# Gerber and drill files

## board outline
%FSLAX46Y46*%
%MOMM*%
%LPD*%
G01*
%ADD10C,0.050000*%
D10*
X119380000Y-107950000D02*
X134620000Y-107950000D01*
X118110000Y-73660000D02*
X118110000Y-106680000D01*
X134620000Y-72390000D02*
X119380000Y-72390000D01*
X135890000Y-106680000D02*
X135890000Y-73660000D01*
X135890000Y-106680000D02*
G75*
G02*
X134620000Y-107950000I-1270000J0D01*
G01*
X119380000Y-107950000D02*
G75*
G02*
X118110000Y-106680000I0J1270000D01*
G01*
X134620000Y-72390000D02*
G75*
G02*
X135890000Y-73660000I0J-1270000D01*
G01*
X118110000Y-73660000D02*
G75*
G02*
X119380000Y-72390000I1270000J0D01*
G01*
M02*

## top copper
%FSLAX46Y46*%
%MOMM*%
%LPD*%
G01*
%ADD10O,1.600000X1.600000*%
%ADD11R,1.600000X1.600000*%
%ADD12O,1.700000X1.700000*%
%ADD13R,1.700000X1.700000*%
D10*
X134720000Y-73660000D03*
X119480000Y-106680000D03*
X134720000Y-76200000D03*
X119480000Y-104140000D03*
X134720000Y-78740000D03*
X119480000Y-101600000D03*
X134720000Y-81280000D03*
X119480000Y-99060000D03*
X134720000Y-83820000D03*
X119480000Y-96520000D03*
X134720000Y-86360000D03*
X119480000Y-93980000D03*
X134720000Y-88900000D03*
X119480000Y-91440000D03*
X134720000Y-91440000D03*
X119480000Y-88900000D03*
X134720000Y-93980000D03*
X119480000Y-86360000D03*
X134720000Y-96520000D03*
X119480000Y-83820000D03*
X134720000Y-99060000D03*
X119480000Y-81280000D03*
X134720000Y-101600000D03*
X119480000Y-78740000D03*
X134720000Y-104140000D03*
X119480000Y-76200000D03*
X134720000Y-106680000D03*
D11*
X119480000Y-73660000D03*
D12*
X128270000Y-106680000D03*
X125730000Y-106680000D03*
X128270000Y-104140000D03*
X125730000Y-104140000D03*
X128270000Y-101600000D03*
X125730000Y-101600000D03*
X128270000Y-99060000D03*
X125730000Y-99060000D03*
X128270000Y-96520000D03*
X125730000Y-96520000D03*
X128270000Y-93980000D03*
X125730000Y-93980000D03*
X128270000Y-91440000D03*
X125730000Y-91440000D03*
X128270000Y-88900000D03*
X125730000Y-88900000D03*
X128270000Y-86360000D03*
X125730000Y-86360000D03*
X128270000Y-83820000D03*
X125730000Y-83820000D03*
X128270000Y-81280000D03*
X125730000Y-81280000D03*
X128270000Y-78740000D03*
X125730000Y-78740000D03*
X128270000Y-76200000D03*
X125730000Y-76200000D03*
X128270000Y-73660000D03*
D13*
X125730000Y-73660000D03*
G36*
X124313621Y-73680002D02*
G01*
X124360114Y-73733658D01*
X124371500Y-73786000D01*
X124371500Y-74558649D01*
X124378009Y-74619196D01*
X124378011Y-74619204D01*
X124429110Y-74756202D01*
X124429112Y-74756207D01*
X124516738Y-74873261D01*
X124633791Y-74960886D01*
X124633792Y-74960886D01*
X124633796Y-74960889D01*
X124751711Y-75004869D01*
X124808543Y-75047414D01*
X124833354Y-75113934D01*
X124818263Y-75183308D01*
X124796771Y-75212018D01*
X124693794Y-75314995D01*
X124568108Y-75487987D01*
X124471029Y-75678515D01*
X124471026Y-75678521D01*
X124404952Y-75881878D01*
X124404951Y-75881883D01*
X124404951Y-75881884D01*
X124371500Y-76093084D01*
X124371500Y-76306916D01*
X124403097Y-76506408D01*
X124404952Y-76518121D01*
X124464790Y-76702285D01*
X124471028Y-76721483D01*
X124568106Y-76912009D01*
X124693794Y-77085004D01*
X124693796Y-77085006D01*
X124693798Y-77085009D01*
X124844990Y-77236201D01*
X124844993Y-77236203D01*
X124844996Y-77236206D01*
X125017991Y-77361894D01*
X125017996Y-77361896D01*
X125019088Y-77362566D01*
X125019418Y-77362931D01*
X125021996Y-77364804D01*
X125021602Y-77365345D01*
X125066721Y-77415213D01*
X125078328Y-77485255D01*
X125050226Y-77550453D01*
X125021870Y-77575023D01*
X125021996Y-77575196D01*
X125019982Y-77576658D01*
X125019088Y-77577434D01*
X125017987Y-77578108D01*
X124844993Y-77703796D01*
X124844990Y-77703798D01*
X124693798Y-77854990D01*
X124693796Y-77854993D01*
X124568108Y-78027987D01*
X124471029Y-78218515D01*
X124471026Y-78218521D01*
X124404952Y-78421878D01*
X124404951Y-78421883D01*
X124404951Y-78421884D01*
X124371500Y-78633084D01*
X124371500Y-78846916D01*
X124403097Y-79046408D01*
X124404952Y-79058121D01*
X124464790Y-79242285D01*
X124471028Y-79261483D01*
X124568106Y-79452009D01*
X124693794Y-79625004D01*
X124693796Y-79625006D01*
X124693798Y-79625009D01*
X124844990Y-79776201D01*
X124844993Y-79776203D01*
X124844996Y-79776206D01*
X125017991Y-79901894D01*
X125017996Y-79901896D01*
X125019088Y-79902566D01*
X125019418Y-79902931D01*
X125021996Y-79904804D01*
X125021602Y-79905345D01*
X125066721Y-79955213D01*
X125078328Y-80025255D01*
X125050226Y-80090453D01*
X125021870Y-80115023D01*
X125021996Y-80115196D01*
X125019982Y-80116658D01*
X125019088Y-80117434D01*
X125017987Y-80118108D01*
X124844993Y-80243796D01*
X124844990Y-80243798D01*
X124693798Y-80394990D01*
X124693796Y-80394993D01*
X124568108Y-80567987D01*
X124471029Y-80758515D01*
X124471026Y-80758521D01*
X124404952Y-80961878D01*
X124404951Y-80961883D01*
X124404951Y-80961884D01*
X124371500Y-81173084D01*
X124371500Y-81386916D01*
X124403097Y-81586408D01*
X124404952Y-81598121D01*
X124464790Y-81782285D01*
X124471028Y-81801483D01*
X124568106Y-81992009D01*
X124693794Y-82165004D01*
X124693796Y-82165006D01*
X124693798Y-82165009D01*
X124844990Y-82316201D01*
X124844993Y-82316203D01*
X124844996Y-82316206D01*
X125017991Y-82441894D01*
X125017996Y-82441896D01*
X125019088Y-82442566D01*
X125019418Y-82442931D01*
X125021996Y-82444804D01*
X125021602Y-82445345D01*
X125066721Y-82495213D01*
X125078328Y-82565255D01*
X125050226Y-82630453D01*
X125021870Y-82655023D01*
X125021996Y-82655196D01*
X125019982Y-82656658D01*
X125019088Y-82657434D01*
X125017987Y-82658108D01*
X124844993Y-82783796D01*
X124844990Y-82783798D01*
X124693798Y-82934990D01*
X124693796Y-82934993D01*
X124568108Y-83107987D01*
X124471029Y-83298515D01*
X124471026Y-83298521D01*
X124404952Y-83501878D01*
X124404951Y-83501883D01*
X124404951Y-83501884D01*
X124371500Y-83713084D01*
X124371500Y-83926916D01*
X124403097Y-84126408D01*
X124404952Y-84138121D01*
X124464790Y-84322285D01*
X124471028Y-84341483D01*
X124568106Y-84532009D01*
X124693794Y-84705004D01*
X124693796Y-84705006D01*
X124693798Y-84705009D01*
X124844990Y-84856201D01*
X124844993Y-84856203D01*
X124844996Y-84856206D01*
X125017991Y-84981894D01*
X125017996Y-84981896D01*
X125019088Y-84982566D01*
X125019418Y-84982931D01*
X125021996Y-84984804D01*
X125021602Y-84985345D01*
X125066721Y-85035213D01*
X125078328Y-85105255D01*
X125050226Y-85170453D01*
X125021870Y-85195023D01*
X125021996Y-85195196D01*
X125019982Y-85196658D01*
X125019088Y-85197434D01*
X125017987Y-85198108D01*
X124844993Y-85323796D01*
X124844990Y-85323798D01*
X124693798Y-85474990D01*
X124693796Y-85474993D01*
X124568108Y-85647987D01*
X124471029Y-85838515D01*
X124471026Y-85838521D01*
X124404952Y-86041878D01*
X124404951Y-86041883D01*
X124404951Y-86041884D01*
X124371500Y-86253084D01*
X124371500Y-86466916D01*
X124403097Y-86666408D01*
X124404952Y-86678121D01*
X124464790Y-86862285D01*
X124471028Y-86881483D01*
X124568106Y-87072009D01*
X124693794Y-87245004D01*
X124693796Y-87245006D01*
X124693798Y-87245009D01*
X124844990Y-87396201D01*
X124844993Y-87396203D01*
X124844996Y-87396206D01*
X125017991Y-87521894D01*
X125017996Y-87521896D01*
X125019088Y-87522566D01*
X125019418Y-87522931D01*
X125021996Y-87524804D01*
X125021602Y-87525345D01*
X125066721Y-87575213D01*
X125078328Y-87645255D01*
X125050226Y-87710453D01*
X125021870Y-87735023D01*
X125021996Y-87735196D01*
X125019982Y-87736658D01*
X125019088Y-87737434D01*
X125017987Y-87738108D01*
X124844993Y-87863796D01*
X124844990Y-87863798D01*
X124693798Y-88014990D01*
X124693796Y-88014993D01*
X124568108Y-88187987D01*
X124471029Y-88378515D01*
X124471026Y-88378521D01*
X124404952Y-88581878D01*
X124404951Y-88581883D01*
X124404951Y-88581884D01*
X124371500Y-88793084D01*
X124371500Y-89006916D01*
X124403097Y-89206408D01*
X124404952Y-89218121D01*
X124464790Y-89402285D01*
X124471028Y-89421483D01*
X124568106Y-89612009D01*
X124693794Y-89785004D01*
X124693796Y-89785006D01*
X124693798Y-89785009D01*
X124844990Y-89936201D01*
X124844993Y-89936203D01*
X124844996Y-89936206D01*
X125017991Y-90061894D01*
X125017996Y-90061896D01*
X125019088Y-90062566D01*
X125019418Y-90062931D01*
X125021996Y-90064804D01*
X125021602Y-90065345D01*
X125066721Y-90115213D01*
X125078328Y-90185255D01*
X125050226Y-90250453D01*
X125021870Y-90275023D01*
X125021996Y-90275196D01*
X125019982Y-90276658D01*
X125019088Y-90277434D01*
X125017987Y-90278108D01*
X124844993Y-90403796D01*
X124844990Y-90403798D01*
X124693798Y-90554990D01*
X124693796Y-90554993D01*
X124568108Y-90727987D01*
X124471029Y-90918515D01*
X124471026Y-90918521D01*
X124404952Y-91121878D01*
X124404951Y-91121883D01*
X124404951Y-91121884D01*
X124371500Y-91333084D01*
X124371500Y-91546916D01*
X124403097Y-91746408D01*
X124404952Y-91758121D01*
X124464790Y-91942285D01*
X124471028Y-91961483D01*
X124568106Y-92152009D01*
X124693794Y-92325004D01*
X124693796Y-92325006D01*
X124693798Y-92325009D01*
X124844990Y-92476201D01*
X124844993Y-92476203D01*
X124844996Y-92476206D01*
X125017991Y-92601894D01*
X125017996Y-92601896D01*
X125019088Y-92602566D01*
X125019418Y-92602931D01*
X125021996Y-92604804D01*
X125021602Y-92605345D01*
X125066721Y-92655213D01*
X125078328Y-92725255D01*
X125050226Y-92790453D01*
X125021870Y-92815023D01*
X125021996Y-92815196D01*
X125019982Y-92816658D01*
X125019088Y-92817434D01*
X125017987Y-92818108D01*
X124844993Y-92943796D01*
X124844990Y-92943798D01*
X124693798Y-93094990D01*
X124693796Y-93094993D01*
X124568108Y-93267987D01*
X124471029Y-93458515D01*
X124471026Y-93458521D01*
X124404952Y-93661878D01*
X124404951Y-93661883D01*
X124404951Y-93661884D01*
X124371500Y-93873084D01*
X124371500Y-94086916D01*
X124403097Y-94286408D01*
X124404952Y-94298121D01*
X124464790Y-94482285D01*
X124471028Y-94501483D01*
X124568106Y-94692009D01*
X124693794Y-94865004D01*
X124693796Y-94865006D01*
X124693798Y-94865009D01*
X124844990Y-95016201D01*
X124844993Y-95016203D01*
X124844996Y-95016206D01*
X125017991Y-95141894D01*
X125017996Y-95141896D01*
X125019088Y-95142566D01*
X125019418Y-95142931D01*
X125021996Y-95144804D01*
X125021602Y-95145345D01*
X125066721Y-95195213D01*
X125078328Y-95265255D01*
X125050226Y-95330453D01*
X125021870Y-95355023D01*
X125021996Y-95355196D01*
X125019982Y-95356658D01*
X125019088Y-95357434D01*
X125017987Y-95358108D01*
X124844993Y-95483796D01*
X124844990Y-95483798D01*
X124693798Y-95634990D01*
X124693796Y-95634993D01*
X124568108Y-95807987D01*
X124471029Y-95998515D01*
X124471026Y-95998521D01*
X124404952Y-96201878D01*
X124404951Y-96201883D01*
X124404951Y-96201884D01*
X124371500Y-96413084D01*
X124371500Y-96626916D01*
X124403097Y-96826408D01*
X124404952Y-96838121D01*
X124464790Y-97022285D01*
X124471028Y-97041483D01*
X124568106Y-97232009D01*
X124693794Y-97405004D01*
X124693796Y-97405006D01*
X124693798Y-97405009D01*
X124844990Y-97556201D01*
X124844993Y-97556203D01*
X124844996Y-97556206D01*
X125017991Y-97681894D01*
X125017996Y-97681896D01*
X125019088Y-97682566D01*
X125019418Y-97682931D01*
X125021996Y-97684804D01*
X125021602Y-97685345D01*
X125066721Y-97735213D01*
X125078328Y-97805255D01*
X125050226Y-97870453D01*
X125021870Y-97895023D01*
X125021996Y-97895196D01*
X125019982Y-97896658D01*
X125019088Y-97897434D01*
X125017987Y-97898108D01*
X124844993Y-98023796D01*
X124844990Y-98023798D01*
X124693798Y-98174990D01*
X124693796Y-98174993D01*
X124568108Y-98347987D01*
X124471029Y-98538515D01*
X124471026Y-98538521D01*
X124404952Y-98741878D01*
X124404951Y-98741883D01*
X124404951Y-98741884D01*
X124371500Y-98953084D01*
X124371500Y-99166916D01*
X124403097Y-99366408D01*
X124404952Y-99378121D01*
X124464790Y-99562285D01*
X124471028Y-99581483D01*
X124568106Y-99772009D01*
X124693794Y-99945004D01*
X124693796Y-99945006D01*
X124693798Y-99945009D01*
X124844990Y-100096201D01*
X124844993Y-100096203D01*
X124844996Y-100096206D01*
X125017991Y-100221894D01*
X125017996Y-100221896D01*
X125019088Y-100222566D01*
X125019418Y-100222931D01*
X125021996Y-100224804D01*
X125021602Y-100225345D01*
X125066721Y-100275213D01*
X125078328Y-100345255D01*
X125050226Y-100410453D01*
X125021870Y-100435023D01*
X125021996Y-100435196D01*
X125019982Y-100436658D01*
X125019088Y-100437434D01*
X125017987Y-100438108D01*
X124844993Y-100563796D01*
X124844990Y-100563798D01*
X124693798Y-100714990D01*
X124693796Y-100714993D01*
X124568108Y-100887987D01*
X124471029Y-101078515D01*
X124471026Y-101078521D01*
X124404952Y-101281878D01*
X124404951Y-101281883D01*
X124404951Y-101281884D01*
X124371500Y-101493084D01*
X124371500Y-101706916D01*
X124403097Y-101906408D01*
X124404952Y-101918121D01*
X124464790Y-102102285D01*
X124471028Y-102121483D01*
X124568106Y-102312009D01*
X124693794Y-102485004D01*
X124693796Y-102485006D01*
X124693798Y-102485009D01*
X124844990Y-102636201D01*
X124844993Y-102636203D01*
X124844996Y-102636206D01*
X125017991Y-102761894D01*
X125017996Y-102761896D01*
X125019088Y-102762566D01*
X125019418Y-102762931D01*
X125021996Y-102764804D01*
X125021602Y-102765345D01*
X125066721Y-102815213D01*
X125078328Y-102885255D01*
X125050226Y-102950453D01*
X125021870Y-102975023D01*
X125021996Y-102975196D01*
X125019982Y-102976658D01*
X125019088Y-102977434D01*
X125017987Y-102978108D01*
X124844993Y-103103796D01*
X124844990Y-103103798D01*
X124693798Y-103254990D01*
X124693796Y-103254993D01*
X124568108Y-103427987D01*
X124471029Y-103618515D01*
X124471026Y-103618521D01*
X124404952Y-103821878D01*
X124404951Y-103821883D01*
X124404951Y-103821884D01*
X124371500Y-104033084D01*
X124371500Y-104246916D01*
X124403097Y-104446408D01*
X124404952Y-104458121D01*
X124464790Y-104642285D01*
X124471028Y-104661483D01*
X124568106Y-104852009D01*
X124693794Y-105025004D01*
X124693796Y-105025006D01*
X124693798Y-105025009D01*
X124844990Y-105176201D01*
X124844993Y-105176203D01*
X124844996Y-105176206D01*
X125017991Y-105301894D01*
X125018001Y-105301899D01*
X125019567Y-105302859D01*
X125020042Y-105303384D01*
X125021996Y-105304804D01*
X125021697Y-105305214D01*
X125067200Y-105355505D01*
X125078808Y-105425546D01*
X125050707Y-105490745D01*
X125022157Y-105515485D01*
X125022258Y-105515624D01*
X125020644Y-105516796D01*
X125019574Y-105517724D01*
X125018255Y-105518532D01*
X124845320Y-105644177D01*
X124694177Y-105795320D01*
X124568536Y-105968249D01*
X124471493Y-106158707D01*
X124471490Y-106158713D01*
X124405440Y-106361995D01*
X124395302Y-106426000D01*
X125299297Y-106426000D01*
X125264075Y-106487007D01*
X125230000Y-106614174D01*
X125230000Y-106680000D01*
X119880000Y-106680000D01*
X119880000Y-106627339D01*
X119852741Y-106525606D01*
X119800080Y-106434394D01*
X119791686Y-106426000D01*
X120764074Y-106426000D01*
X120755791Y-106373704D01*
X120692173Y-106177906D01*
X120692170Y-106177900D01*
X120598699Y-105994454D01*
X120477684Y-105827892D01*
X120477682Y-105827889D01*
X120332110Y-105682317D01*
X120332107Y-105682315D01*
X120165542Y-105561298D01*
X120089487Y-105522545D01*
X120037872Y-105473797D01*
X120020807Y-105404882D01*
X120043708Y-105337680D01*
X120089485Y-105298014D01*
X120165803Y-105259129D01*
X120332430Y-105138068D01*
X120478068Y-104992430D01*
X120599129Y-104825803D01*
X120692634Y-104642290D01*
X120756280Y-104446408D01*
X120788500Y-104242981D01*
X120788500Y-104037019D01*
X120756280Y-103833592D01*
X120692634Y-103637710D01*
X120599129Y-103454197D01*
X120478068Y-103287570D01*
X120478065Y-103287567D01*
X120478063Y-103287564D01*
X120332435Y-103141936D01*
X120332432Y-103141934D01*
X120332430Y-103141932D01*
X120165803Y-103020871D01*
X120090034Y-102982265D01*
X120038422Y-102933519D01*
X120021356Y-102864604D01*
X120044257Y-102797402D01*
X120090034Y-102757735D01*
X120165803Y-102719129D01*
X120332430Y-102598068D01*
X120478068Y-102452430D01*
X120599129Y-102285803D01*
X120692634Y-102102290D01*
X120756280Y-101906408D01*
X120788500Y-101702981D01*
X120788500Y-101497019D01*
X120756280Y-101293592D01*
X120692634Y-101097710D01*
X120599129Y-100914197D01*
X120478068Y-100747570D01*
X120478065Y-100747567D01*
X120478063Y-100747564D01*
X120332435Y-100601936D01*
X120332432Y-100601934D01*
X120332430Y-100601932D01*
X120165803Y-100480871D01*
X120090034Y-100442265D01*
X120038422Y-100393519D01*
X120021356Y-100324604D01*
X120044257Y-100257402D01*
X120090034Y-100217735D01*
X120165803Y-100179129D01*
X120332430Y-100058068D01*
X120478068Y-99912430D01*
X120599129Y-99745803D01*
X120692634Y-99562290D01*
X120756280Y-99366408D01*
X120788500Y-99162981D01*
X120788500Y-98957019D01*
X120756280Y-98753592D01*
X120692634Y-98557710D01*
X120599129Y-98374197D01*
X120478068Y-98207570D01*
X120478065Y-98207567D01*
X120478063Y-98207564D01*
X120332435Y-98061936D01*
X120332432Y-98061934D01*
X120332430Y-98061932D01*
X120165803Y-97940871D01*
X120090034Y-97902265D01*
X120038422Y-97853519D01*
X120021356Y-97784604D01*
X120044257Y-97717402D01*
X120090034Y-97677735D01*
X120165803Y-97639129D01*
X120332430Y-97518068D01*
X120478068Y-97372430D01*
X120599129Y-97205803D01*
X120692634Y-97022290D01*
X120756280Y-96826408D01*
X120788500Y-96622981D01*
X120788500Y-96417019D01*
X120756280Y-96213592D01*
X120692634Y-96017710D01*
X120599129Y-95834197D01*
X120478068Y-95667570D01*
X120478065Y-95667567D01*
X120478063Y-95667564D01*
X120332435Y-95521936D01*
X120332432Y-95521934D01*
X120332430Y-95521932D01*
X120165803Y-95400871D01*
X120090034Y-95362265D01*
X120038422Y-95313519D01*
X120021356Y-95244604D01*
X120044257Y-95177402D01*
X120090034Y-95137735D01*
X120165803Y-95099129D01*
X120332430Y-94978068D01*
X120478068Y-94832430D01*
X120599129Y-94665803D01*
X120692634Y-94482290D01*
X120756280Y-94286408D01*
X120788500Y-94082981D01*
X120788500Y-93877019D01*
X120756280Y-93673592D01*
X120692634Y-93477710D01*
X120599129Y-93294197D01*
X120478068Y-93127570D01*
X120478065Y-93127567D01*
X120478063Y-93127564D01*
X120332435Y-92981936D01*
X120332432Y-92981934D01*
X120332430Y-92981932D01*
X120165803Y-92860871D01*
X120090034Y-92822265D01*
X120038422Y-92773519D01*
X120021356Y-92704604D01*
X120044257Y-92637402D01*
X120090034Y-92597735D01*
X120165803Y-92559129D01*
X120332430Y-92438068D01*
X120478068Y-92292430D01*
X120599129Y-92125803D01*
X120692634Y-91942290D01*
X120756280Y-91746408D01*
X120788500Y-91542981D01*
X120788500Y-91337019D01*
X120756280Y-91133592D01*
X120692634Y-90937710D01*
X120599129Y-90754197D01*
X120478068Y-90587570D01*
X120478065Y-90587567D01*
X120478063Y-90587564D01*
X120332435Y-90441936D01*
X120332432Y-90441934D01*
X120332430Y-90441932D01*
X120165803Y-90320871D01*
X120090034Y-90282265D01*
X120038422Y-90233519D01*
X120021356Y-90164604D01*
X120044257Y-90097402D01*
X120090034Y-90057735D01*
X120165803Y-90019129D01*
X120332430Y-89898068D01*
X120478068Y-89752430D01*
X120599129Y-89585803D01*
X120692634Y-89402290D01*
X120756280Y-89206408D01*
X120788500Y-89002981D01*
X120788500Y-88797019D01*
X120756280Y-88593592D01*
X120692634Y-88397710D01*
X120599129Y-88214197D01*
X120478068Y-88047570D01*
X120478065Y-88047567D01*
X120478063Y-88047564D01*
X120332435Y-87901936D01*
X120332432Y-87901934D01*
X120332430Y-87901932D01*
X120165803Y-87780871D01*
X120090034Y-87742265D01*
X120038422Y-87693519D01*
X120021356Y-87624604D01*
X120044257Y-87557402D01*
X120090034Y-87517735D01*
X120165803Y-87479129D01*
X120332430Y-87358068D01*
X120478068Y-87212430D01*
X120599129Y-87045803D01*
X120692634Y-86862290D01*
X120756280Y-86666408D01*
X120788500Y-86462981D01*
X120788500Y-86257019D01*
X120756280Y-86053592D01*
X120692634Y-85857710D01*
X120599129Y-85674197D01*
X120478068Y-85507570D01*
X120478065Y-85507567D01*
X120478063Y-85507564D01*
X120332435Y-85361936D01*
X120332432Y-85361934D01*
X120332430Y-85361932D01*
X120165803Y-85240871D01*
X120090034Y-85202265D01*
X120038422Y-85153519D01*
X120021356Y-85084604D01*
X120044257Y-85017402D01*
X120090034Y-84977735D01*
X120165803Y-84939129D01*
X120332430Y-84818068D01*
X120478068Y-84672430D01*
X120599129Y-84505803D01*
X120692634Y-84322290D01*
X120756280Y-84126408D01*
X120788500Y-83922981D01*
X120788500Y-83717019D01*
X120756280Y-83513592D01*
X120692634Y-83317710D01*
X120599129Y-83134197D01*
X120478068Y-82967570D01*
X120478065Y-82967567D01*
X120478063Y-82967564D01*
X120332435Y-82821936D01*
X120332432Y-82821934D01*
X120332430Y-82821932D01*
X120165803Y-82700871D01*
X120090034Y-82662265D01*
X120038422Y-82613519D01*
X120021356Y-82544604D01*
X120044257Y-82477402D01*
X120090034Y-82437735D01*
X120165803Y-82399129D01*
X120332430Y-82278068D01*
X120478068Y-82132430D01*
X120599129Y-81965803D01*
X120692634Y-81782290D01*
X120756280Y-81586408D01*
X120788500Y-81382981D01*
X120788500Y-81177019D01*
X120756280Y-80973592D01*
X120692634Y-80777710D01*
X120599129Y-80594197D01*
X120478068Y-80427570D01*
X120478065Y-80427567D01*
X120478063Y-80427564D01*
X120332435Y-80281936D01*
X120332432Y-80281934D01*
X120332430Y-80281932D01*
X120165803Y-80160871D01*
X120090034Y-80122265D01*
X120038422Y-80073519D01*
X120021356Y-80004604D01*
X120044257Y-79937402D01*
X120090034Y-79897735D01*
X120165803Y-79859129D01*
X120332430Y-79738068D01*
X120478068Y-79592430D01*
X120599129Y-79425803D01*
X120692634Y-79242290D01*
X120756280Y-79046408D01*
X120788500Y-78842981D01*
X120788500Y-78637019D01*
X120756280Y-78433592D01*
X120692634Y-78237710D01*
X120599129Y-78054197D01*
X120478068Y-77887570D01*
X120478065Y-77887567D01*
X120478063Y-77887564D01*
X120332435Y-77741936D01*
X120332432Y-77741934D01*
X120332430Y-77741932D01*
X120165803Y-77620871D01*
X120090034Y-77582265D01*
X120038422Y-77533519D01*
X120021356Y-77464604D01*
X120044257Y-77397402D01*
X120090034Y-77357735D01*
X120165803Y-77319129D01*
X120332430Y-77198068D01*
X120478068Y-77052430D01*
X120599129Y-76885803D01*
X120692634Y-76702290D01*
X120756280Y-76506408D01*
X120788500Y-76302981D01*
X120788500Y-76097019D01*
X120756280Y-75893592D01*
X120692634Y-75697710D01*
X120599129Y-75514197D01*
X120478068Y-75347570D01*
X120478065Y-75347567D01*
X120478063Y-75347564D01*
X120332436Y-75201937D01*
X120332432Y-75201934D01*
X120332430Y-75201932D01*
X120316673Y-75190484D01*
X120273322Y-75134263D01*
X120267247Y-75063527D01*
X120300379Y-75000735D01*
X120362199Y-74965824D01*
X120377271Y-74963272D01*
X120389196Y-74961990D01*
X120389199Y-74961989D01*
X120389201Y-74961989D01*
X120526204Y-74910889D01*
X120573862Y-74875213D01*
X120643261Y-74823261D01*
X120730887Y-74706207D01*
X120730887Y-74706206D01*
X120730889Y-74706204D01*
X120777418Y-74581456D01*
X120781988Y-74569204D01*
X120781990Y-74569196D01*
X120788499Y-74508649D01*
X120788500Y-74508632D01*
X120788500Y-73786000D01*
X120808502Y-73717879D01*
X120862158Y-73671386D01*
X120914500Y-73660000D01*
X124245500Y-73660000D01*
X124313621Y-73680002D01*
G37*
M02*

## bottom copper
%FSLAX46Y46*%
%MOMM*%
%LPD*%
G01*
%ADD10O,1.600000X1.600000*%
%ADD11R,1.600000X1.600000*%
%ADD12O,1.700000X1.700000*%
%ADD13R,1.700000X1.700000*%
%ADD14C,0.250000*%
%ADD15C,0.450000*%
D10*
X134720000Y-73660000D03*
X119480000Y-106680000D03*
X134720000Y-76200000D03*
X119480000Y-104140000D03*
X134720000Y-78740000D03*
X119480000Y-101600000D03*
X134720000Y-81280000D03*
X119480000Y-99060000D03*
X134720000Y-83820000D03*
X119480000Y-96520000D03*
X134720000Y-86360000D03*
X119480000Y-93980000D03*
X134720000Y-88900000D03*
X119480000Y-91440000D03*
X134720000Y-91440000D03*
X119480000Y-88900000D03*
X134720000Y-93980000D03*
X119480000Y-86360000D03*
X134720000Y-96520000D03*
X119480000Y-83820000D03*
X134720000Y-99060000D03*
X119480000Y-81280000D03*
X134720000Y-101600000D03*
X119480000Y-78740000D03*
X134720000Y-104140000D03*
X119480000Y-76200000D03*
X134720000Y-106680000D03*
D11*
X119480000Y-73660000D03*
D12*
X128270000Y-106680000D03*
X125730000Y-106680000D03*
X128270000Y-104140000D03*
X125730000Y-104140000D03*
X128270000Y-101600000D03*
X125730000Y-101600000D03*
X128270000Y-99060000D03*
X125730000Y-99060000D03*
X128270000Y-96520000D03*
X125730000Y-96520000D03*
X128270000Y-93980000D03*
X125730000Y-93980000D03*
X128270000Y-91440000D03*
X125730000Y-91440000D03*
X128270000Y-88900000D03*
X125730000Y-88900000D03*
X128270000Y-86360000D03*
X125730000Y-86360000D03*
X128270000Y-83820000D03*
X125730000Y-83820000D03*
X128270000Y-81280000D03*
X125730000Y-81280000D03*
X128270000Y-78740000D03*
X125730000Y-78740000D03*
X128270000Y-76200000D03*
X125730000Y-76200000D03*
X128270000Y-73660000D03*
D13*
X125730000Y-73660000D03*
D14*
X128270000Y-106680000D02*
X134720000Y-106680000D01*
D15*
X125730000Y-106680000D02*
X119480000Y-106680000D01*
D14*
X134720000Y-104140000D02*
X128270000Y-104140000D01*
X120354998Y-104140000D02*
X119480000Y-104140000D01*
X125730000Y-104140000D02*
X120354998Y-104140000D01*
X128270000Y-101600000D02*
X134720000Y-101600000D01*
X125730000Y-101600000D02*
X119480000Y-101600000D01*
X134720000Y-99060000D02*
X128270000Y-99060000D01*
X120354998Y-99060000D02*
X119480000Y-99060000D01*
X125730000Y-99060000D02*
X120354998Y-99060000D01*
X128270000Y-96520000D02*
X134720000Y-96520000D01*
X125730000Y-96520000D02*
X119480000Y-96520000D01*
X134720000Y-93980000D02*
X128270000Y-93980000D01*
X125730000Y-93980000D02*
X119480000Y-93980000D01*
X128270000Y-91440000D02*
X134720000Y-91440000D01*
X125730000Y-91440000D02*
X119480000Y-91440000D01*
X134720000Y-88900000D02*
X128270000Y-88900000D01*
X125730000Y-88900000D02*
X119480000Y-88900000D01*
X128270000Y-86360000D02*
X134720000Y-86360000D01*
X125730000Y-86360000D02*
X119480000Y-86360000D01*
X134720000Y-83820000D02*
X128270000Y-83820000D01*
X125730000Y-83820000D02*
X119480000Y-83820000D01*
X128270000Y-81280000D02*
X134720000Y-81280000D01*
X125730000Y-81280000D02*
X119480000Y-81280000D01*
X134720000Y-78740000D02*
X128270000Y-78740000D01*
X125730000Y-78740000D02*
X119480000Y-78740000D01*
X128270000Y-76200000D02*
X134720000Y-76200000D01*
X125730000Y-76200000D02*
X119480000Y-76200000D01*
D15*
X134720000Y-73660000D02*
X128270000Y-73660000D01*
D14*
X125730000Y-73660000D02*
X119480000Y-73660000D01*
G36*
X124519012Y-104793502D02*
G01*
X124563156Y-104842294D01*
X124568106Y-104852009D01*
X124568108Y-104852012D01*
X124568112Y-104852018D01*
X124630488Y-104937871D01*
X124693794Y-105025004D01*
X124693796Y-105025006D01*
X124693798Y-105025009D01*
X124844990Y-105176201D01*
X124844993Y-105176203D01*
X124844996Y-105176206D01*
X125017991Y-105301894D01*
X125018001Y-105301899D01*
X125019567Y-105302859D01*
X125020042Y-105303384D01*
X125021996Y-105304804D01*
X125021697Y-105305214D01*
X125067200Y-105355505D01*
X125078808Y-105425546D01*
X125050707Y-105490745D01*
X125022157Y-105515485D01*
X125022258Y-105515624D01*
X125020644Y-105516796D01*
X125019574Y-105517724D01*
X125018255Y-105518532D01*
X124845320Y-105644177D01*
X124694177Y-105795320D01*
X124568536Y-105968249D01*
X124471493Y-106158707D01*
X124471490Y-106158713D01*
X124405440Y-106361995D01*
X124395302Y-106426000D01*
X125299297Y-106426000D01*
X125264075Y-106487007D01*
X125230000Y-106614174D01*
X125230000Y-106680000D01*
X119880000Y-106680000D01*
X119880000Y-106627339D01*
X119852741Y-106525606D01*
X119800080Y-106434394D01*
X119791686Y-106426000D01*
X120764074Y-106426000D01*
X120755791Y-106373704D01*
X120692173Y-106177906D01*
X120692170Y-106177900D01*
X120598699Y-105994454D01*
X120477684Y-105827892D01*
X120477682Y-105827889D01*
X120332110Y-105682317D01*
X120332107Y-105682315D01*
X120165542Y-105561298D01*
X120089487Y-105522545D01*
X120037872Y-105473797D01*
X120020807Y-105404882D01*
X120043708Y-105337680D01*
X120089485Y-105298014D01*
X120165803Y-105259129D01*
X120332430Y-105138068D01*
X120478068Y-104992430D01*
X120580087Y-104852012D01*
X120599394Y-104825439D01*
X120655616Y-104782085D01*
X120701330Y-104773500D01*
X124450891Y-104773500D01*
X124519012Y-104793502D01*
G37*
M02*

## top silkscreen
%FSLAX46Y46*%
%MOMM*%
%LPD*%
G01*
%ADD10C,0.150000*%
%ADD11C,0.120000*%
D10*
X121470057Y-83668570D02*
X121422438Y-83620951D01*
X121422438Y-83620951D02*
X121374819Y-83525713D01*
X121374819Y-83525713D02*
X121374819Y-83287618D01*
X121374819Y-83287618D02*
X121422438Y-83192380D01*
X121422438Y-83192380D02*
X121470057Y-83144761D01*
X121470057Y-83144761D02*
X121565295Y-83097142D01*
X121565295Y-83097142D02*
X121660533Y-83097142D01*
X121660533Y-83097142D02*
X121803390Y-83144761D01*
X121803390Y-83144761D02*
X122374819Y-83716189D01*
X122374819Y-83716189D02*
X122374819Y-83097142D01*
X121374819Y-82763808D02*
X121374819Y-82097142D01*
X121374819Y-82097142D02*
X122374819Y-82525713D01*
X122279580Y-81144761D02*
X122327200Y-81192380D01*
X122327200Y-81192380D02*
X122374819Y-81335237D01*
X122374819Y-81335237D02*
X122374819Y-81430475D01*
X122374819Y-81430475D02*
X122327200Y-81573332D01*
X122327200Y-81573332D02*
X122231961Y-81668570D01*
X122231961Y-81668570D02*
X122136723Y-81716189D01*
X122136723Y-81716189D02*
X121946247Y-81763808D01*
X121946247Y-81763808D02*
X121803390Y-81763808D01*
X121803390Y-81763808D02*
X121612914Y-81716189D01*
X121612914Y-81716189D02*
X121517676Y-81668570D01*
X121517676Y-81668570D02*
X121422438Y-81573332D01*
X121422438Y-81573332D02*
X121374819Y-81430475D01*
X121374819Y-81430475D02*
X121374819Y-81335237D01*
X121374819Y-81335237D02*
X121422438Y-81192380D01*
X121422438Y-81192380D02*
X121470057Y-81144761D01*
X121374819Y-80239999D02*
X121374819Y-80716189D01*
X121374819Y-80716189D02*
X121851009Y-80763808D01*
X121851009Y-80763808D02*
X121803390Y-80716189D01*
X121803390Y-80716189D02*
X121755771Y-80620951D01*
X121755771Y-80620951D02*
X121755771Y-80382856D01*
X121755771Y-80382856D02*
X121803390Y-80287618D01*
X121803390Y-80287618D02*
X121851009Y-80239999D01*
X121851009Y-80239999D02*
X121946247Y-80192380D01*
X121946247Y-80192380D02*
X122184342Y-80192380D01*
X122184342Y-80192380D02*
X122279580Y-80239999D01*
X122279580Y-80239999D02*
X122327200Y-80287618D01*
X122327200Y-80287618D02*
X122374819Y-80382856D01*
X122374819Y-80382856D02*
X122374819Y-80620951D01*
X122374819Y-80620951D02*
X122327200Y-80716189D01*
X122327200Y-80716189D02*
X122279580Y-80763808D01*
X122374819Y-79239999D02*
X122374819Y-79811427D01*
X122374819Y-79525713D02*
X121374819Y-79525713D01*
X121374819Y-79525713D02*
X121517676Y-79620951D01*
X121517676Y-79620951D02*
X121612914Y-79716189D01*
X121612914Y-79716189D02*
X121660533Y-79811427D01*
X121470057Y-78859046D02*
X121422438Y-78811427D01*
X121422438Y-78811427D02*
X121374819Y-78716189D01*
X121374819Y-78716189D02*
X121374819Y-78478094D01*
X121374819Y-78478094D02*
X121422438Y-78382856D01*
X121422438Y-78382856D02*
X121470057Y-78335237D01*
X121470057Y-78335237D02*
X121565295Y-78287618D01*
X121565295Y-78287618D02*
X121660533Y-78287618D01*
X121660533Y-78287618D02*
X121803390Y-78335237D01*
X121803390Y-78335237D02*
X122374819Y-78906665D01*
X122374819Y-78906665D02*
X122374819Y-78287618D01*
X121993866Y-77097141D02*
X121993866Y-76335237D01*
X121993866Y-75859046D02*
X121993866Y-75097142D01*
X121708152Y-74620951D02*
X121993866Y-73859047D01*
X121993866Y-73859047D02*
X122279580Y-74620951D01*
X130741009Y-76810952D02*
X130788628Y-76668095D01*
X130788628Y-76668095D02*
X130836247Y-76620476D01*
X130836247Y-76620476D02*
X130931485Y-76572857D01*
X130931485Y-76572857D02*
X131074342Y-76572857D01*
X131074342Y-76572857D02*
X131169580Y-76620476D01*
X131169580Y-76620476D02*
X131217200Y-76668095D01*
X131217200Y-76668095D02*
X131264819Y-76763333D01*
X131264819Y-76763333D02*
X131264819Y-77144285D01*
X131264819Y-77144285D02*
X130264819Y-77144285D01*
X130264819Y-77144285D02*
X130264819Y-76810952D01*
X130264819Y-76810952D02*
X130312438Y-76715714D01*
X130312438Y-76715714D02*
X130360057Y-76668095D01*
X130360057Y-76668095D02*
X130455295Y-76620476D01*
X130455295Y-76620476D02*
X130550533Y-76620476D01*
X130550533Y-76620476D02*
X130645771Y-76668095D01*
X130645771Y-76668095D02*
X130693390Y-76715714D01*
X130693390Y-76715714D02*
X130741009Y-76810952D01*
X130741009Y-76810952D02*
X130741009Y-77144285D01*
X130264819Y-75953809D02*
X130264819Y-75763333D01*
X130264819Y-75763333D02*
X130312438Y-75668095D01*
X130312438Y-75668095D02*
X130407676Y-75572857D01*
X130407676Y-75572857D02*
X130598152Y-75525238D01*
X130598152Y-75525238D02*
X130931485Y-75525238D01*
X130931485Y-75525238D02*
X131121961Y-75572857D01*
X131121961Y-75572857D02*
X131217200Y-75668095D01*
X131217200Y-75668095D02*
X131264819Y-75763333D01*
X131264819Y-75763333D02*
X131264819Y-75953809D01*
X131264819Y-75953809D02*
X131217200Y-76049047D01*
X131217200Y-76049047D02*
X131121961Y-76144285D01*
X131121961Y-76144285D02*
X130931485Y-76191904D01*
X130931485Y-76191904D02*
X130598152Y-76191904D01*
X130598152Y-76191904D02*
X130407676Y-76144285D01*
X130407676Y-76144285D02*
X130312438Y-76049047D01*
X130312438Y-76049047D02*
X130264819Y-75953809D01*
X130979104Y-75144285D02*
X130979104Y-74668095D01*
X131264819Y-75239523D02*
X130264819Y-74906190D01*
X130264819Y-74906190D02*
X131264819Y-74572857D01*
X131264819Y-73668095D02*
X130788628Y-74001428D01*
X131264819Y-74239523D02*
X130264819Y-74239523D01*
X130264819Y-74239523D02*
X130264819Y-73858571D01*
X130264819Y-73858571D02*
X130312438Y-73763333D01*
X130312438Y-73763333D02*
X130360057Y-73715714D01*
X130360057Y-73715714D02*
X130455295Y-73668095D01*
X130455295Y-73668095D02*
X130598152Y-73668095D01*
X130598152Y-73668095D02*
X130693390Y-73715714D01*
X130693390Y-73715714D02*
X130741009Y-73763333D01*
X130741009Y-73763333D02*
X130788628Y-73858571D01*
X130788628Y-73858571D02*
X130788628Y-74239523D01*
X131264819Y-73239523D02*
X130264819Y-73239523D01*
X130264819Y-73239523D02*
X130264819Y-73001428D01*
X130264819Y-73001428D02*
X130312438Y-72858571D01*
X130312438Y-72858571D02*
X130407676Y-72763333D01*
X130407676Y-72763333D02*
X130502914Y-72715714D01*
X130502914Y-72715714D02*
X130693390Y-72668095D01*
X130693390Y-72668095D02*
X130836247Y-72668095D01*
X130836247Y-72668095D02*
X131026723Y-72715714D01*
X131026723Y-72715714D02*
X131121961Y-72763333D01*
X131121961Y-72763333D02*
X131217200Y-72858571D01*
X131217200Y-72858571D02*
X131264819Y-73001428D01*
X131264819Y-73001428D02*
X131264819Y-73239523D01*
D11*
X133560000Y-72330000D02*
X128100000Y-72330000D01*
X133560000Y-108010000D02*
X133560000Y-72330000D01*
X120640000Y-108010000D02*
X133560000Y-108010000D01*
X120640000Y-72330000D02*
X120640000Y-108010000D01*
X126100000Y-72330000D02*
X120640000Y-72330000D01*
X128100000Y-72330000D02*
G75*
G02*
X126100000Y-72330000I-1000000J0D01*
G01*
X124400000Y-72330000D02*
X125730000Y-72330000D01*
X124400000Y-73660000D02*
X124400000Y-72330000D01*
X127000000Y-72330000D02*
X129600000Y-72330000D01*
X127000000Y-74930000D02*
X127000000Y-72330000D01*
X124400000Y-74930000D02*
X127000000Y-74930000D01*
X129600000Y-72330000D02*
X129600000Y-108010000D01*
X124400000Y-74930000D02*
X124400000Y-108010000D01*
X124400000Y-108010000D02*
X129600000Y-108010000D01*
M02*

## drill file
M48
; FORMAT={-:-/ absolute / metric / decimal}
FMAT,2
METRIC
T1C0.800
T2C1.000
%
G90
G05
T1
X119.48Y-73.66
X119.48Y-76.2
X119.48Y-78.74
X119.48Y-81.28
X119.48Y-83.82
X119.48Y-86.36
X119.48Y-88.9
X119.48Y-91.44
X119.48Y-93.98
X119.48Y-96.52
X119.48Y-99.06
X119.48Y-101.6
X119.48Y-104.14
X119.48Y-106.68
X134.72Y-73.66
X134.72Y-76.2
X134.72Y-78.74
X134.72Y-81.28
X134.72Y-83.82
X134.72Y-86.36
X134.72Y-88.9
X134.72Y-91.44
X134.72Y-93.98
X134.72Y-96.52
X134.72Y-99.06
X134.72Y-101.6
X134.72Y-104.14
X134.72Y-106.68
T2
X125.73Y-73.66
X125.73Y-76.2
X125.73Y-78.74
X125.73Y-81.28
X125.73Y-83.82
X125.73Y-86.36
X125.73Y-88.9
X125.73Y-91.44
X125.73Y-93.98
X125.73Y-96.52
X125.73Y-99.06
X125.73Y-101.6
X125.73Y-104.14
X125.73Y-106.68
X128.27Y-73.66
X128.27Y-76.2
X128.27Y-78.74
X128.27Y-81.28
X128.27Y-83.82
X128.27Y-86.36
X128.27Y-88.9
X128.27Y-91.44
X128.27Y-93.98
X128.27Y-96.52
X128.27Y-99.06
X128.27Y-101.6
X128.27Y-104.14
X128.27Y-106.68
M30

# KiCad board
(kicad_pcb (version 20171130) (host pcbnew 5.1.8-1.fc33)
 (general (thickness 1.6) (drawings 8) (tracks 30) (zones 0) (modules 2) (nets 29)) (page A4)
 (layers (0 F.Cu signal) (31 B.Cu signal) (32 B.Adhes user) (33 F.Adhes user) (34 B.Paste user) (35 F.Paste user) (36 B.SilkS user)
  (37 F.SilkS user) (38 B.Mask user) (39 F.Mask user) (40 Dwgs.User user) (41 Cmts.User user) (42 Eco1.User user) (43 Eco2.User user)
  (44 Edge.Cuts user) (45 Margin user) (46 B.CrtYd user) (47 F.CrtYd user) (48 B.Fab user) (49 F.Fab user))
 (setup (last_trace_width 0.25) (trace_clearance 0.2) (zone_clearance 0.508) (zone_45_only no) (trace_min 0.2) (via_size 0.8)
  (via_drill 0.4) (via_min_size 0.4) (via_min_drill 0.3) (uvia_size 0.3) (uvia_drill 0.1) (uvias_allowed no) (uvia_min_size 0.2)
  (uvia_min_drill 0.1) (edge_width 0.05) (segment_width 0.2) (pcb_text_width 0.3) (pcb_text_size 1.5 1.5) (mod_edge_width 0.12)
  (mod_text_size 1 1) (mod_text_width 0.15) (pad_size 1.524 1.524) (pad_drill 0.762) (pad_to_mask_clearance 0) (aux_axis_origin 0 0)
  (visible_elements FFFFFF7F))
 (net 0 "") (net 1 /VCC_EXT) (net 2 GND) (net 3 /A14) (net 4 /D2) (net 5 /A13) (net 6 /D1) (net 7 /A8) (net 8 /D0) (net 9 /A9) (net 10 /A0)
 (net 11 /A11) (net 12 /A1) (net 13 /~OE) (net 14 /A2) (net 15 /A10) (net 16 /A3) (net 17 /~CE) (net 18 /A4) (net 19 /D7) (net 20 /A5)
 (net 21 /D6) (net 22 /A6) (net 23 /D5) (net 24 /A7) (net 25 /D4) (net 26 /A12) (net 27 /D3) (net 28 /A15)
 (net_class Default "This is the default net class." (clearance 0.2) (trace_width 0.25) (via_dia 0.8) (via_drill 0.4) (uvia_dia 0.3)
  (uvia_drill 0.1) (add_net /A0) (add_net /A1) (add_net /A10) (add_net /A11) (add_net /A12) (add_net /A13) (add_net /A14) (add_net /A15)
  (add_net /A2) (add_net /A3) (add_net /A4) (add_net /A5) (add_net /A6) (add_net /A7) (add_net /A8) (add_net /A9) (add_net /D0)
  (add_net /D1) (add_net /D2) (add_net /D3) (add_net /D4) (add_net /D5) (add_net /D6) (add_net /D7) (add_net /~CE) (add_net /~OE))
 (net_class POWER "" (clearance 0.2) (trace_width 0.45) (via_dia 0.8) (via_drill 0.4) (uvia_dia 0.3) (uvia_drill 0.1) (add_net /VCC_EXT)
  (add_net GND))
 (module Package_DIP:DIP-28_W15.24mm (layer F.Cu) (at 119.48 73.66)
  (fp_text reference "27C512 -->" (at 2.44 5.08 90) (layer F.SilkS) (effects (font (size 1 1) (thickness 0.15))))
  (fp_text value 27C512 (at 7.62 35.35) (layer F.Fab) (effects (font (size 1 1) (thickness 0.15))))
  (fp_line (start 14.08 -1.33) (end 8.62 -1.33) (layer F.SilkS) (width 0.12))
  (fp_line (start 14.08 34.35) (end 14.08 -1.33) (layer F.SilkS) (width 0.12))
  (fp_line (start 1.16 34.35) (end 14.08 34.35) (layer F.SilkS) (width 0.12))
  (fp_line (start 1.16 -1.33) (end 1.16 34.35) (layer F.SilkS) (width 0.12))
  (fp_line (start 6.62 -1.33) (end 1.16 -1.33) (layer F.SilkS) (width 0.12))
  (fp_arc (start 7.62 -1.33) (end 6.62 -1.33) (angle -180) (layer F.SilkS) (width 0.12))
  (pad 28 thru_hole oval (at 15.24 0) (size 1.6 1.6) (drill 0.8) (layers *.Cu *.Mask) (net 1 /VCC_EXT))
  (pad 14 thru_hole oval (at 0 33.02) (size 1.6 1.6) (drill 0.8) (layers *.Cu *.Mask) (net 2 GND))
  (pad 27 thru_hole oval (at 15.24 2.54) (size 1.6 1.6) (drill 0.8) (layers *.Cu *.Mask) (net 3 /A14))
  (pad 13 thru_hole oval (at 0 30.48) (size 1.6 1.6) (drill 0.8) (layers *.Cu *.Mask) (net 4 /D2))
  (pad 26 thru_hole oval (at 15.24 5.08) (size 1.6 1.6) (drill 0.8) (layers *.Cu *.Mask) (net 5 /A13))
  (pad 12 thru_hole oval (at 0 27.94) (size 1.6 1.6) (drill 0.8) (layers *.Cu *.Mask) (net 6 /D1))
  (pad 25 thru_hole oval (at 15.24 7.62) (size 1.6 1.6) (drill 0.8) (layers *.Cu *.Mask) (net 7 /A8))
  (pad 11 thru_hole oval (at 0 25.4) (size 1.6 1.6) (drill 0.8) (layers *.Cu *.Mask) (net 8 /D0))
  (pad 24 thru_hole oval (at 15.24 10.16) (size 1.6 1.6) (drill 0.8) (layers *.Cu *.Mask) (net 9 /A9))
  (pad 10 thru_hole oval (at 0 22.86) (size 1.6 1.6) (drill 0.8) (layers *.Cu *.Mask) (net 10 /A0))
  (pad 23 thru_hole oval (at 15.24 12.7) (size 1.6 1.6) (drill 0.8) (layers *.Cu *.Mask) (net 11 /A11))
  (pad 9 thru_hole oval (at 0 20.32) (size 1.6 1.6) (drill 0.8) (layers *.Cu *.Mask) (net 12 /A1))
  (pad 22 thru_hole oval (at 15.24 15.24) (size 1.6 1.6) (drill 0.8) (layers *.Cu *.Mask) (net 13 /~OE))
  (pad 8 thru_hole oval (at 0 17.78) (size 1.6 1.6) (drill 0.8) (layers *.Cu *.Mask) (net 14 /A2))
  (pad 21 thru_hole oval (at 15.24 17.78) (size 1.6 1.6) (drill 0.8) (layers *.Cu *.Mask) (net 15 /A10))
  (pad 7 thru_hole oval (at 0 15.24) (size 1.6 1.6) (drill 0.8) (layers *.Cu *.Mask) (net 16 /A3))
  (pad 20 thru_hole oval (at 15.24 20.32) (size 1.6 1.6) (drill 0.8) (layers *.Cu *.Mask) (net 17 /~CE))
  (pad 6 thru_hole oval (at 0 12.7) (size 1.6 1.6) (drill 0.8) (layers *.Cu *.Mask) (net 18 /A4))
  (pad 19 thru_hole oval (at 15.24 22.86) (size 1.6 1.6) (drill 0.8) (layers *.Cu *.Mask) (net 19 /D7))
  (pad 5 thru_hole oval (at 0 10.16) (size 1.6 1.6) (drill 0.8) (layers *.Cu *.Mask) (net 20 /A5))
  (pad 18 thru_hole oval (at 15.24 25.4) (size 1.6 1.6) (drill 0.8) (layers *.Cu *.Mask) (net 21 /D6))
  (pad 4 thru_hole oval (at 0 7.62) (size 1.6 1.6) (drill 0.8) (layers *.Cu *.Mask) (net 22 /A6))
  (pad 17 thru_hole oval (at 15.24 27.94) (size 1.6 1.6) (drill 0.8) (layers *.Cu *.Mask) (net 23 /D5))
  (pad 3 thru_hole oval (at 0 5.08) (size 1.6 1.6) (drill 0.8) (layers *.Cu *.Mask) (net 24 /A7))
  (pad 16 thru_hole oval (at 15.24 30.48) (size 1.6 1.6) (drill 0.8) (layers *.Cu *.Mask) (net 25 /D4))
  (pad 2 thru_hole oval (at 0 2.54) (size 1.6 1.6) (drill 0.8) (layers *.Cu *.Mask) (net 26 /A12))
  (pad 15 thru_hole oval (at 15.24 33.02) (size 1.6 1.6) (drill 0.8) (layers *.Cu *.Mask) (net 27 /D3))
  (pad 1 thru_hole rect (at 0 0) (size 1.6 1.6) (drill 0.8) (layers *.Cu *.Mask) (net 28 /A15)))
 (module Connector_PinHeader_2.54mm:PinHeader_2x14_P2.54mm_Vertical (layer F.Cu) (at 125.73 73.66)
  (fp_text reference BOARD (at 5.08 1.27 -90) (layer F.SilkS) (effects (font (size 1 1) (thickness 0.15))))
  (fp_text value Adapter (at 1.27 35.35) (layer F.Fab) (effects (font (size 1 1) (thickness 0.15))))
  (fp_line (start -1.33 -1.33) (end 0 -1.33) (layer F.SilkS) (width 0.12))
  (fp_line (start -1.33 0) (end -1.33 -1.33) (layer F.SilkS) (width 0.12))
  (fp_line (start 1.27 -1.33) (end 3.87 -1.33) (layer F.SilkS) (width 0.12))
  (fp_line (start 1.27 1.27) (end 1.27 -1.33) (layer F.SilkS) (width 0.12))
  (fp_line (start -1.33 1.27) (end 1.27 1.27) (layer F.SilkS) (width 0.12))
  (fp_line (start 3.87 -1.33) (end 3.87 34.35) (layer F.SilkS) (width 0.12))
  (fp_line (start -1.33 1.27) (end -1.33 34.35) (layer F.SilkS) (width 0.12))
  (fp_line (start -1.33 34.35) (end 3.87 34.35) (layer F.SilkS) (width 0.12))
  (pad 28 thru_hole oval (at 2.54 33.02) (size 1.7 1.7) (drill 1) (layers *.Cu *.Mask) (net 27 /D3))
  (pad 27 thru_hole oval (at 0 33.02) (size 1.7 1.7) (drill 1) (layers *.Cu *.Mask) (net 2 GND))
  (pad 26 thru_hole oval (at 2.54 30.48) (size 1.7 1.7) (drill 1) (layers *.Cu *.Mask) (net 25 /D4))
  (pad 25 thru_hole oval (at 0 30.48) (size 1.7 1.7) (drill 1) (layers *.Cu *.Mask) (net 4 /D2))
  (pad 24 thru_hole oval (at 2.54 27.94) (size 1.7 1.7) (drill 1) (layers *.Cu *.Mask) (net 23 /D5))
  (pad 23 thru_hole oval (at 0 27.94) (size 1.7 1.7) (drill 1) (layers *.Cu *.Mask) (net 6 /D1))
  (pad 22 thru_hole oval (at 2.54 25.4) (size 1.7 1.7) (drill 1) (layers *.Cu *.Mask) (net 21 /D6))
  (pad 21 thru_hole oval (at 0 25.4) (size 1.7 1.7) (drill 1) (layers *.Cu *.Mask) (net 8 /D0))
  (pad 20 thru_hole oval (at 2.54 22.86) (size 1.7 1.7) (drill 1) (layers *.Cu *.Mask) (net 19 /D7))
  (pad 19 thru_hole oval (at 0 22.86) (size 1.7 1.7) (drill 1) (layers *.Cu *.Mask) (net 10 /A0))
  (pad 18 thru_hole oval (at 2.54 20.32) (size 1.7 1.7) (drill 1) (layers *.Cu *.Mask) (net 17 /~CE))
  (pad 17 thru_hole oval (at 0 20.32) (size 1.7 1.7) (drill 1) (layers *.Cu *.Mask) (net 12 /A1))
  (pad 16 thru_hole oval (at 2.54 17.78) (size 1.7 1.7) (drill 1) (layers *.Cu *.Mask) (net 15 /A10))
  (pad 15 thru_hole oval (at 0 17.78) (size 1.7 1.7) (drill 1) (layers *.Cu *.Mask) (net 14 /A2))
  (pad 14 thru_hole oval (at 2.54 15.24) (size 1.7 1.7) (drill 1) (layers *.Cu *.Mask) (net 13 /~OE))
  (pad 13 thru_hole oval (at 0 15.24) (size 1.7 1.7) (drill 1) (layers *.Cu *.Mask) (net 16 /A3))
  (pad 12 thru_hole oval (at 2.54 12.7) (size 1.7 1.7) (drill 1) (layers *.Cu *.Mask) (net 11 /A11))
  (pad 11 thru_hole oval (at 0 12.7) (size 1.7 1.7) (drill 1) (layers *.Cu *.Mask) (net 18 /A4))
  (pad 10 thru_hole oval (at 2.54 10.16) (size 1.7 1.7) (drill 1) (layers *.Cu *.Mask) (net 9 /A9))
  (pad 9 thru_hole oval (at 0 10.16) (size 1.7 1.7) (drill 1) (layers *.Cu *.Mask) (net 20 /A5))
  (pad 8 thru_hole oval (at 2.54 7.62) (size 1.7 1.7) (drill 1) (layers *.Cu *.Mask) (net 7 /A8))
  (pad 7 thru_hole oval (at 0 7.62) (size 1.7 1.7) (drill 1) (layers *.Cu *.Mask) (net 22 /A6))
  (pad 6 thru_hole oval (at 2.54 5.08) (size 1.7 1.7) (drill 1) (layers *.Cu *.Mask) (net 5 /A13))
  (pad 5 thru_hole oval (at 0 5.08) (size 1.7 1.7) (drill 1) (layers *.Cu *.Mask) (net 24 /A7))
  (pad 4 thru_hole oval (at 2.54 2.54) (size 1.7 1.7) (drill 1) (layers *.Cu *.Mask) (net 3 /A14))
  (pad 3 thru_hole oval (at 0 2.54) (size 1.7 1.7) (drill 1) (layers *.Cu *.Mask) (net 26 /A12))
  (pad 2 thru_hole oval (at 2.54 0) (size 1.7 1.7) (drill 1) (layers *.Cu *.Mask) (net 1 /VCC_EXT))
  (pad 1 thru_hole rect (at 0 0) (size 1.7 1.7) (drill 1) (layers *.Cu *.Mask) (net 28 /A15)))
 (gr_line (start 119.38 107.95) (end 134.62 107.95) (layer Edge.Cuts) (width 0.05))
 (gr_line (start 118.11 73.66) (end 118.11 106.68) (layer Edge.Cuts) (width 0.05))
 (gr_line (start 134.62 72.39) (end 119.38 72.39) (layer Edge.Cuts) (width 0.05))
 (gr_line (start 135.89 106.68) (end 135.89 73.66) (layer Edge.Cuts) (width 0.05))
 (gr_arc (start 134.62 106.68) (end 134.62 107.95) (angle -90) (layer Edge.Cuts) (width 0.05))
 (gr_arc (start 119.38 106.68) (end 118.11 106.68) (angle -90) (layer Edge.Cuts) (width 0.05))
 (gr_arc (start 134.62 73.66) (end 135.89 73.66) (angle -90) (layer Edge.Cuts) (width 0.05))
 (gr_arc (start 119.38 73.66) (end 119.38 72.39) (angle -90) (layer Edge.Cuts) (width 0.05))
 (segment (start 128.27 106.68) (end 134.72 106.68) (width 0.25) (layer B.Cu) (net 27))
 (segment (start 125.73 106.68) (end 119.48 106.68) (width 0.45) (layer B.Cu) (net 2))
 (segment (start 134.72 104.14) (end 128.27 104.14) (width 0.25) (layer B.Cu) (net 25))
 (segment (start 120.354998 104.14) (end 119.48 104.14) (width 0.25) (layer B.Cu) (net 4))
 (segment (start 125.73 104.14) (end 120.354998 104.14) (width 0.25) (layer B.Cu) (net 4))
 (segment (start 128.27 101.6) (end 134.72 101.6) (width 0.25) (layer B.Cu) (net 23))
 (segment (start 125.73 101.6) (end 119.48 101.6) (width 0.25) (layer B.Cu) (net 6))
 (segment (start 134.72 99.06) (end 128.27 99.06) (width 0.25) (layer B.Cu) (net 21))
 (segment (start 120.354998 99.06) (end 119.48 99.06) (width 0.25) (layer B.Cu) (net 8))
 (segment (start 125.73 99.06) (end 120.354998 99.06) (width 0.25) (layer B.Cu) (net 8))
 (segment (start 128.27 96.52) (end 134.72 96.52) (width 0.25) (layer B.Cu) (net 19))
 (segment (start 125.73 96.52) (end 119.48 96.52) (width 0.25) (layer B.Cu) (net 10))
 (segment (start 134.72 93.98) (end 128.27 93.98) (width 0.25) (layer B.Cu) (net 17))
 (segment (start 125.73 93.98) (end 119.48 93.98) (width 0.25) (layer B.Cu) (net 12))
 (segment (start 128.27 91.44) (end 134.72 91.44) (width 0.25) (layer B.Cu) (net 15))
 (segment (start 125.73 91.44) (end 119.48 91.44) (width 0.25) (layer B.Cu) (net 14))
 (segment (start 134.72 88.9) (end 128.27 88.9) (width 0.25) (layer B.Cu) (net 13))
 (segment (start 125.73 88.9) (end 119.48 88.9) (width 0.25) (layer B.Cu) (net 16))
 (segment (start 128.27 86.36) (end 134.72 86.36) (width 0.25) (layer B.Cu) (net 11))
 (segment (start 125.73 86.36) (end 119.48 86.36) (width 0.25) (layer B.Cu) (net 18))
 (segment (start 134.72 83.82) (end 128.27 83.82) (width 0.25) (layer B.Cu) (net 9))
 (segment (start 125.73 83.82) (end 119.48 83.82) (width 0.25) (layer B.Cu) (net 20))
 (segment (start 128.27 81.28) (end 134.72 81.28) (width 0.25) (layer B.Cu) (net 7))
 (segment (start 125.73 81.28) (end 119.48 81.28) (width 0.25) (layer B.Cu) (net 22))
 (segment (start 134.72 78.74) (end 128.27 78.74) (width 0.25) (layer B.Cu) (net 5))
 (segment (start 125.73 78.74) (end 119.48 78.74) (width 0.25) (layer B.Cu) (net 24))
 (segment (start 128.27 76.2) (end 134.72 76.2) (width 0.25) (layer B.Cu) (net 3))
 (segment (start 125.73 76.2) (end 119.48 76.2) (width 0.25) (layer B.Cu) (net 26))
 (segment (start 134.72 73.66) (end 128.27 73.66) (width 0.45) (layer B.Cu) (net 1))
 (segment (start 125.73 73.66) (end 119.48 73.66) (width 0.25) (layer B.Cu) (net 28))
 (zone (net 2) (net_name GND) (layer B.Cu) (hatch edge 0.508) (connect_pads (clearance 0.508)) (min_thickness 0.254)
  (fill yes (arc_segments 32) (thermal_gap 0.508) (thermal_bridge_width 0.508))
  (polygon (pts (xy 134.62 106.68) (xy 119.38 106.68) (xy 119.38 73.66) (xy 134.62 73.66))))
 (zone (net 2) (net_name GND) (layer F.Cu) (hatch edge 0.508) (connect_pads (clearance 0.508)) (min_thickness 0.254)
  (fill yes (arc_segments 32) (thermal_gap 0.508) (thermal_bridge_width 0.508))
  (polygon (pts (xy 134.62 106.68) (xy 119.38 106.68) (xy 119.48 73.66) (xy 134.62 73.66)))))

